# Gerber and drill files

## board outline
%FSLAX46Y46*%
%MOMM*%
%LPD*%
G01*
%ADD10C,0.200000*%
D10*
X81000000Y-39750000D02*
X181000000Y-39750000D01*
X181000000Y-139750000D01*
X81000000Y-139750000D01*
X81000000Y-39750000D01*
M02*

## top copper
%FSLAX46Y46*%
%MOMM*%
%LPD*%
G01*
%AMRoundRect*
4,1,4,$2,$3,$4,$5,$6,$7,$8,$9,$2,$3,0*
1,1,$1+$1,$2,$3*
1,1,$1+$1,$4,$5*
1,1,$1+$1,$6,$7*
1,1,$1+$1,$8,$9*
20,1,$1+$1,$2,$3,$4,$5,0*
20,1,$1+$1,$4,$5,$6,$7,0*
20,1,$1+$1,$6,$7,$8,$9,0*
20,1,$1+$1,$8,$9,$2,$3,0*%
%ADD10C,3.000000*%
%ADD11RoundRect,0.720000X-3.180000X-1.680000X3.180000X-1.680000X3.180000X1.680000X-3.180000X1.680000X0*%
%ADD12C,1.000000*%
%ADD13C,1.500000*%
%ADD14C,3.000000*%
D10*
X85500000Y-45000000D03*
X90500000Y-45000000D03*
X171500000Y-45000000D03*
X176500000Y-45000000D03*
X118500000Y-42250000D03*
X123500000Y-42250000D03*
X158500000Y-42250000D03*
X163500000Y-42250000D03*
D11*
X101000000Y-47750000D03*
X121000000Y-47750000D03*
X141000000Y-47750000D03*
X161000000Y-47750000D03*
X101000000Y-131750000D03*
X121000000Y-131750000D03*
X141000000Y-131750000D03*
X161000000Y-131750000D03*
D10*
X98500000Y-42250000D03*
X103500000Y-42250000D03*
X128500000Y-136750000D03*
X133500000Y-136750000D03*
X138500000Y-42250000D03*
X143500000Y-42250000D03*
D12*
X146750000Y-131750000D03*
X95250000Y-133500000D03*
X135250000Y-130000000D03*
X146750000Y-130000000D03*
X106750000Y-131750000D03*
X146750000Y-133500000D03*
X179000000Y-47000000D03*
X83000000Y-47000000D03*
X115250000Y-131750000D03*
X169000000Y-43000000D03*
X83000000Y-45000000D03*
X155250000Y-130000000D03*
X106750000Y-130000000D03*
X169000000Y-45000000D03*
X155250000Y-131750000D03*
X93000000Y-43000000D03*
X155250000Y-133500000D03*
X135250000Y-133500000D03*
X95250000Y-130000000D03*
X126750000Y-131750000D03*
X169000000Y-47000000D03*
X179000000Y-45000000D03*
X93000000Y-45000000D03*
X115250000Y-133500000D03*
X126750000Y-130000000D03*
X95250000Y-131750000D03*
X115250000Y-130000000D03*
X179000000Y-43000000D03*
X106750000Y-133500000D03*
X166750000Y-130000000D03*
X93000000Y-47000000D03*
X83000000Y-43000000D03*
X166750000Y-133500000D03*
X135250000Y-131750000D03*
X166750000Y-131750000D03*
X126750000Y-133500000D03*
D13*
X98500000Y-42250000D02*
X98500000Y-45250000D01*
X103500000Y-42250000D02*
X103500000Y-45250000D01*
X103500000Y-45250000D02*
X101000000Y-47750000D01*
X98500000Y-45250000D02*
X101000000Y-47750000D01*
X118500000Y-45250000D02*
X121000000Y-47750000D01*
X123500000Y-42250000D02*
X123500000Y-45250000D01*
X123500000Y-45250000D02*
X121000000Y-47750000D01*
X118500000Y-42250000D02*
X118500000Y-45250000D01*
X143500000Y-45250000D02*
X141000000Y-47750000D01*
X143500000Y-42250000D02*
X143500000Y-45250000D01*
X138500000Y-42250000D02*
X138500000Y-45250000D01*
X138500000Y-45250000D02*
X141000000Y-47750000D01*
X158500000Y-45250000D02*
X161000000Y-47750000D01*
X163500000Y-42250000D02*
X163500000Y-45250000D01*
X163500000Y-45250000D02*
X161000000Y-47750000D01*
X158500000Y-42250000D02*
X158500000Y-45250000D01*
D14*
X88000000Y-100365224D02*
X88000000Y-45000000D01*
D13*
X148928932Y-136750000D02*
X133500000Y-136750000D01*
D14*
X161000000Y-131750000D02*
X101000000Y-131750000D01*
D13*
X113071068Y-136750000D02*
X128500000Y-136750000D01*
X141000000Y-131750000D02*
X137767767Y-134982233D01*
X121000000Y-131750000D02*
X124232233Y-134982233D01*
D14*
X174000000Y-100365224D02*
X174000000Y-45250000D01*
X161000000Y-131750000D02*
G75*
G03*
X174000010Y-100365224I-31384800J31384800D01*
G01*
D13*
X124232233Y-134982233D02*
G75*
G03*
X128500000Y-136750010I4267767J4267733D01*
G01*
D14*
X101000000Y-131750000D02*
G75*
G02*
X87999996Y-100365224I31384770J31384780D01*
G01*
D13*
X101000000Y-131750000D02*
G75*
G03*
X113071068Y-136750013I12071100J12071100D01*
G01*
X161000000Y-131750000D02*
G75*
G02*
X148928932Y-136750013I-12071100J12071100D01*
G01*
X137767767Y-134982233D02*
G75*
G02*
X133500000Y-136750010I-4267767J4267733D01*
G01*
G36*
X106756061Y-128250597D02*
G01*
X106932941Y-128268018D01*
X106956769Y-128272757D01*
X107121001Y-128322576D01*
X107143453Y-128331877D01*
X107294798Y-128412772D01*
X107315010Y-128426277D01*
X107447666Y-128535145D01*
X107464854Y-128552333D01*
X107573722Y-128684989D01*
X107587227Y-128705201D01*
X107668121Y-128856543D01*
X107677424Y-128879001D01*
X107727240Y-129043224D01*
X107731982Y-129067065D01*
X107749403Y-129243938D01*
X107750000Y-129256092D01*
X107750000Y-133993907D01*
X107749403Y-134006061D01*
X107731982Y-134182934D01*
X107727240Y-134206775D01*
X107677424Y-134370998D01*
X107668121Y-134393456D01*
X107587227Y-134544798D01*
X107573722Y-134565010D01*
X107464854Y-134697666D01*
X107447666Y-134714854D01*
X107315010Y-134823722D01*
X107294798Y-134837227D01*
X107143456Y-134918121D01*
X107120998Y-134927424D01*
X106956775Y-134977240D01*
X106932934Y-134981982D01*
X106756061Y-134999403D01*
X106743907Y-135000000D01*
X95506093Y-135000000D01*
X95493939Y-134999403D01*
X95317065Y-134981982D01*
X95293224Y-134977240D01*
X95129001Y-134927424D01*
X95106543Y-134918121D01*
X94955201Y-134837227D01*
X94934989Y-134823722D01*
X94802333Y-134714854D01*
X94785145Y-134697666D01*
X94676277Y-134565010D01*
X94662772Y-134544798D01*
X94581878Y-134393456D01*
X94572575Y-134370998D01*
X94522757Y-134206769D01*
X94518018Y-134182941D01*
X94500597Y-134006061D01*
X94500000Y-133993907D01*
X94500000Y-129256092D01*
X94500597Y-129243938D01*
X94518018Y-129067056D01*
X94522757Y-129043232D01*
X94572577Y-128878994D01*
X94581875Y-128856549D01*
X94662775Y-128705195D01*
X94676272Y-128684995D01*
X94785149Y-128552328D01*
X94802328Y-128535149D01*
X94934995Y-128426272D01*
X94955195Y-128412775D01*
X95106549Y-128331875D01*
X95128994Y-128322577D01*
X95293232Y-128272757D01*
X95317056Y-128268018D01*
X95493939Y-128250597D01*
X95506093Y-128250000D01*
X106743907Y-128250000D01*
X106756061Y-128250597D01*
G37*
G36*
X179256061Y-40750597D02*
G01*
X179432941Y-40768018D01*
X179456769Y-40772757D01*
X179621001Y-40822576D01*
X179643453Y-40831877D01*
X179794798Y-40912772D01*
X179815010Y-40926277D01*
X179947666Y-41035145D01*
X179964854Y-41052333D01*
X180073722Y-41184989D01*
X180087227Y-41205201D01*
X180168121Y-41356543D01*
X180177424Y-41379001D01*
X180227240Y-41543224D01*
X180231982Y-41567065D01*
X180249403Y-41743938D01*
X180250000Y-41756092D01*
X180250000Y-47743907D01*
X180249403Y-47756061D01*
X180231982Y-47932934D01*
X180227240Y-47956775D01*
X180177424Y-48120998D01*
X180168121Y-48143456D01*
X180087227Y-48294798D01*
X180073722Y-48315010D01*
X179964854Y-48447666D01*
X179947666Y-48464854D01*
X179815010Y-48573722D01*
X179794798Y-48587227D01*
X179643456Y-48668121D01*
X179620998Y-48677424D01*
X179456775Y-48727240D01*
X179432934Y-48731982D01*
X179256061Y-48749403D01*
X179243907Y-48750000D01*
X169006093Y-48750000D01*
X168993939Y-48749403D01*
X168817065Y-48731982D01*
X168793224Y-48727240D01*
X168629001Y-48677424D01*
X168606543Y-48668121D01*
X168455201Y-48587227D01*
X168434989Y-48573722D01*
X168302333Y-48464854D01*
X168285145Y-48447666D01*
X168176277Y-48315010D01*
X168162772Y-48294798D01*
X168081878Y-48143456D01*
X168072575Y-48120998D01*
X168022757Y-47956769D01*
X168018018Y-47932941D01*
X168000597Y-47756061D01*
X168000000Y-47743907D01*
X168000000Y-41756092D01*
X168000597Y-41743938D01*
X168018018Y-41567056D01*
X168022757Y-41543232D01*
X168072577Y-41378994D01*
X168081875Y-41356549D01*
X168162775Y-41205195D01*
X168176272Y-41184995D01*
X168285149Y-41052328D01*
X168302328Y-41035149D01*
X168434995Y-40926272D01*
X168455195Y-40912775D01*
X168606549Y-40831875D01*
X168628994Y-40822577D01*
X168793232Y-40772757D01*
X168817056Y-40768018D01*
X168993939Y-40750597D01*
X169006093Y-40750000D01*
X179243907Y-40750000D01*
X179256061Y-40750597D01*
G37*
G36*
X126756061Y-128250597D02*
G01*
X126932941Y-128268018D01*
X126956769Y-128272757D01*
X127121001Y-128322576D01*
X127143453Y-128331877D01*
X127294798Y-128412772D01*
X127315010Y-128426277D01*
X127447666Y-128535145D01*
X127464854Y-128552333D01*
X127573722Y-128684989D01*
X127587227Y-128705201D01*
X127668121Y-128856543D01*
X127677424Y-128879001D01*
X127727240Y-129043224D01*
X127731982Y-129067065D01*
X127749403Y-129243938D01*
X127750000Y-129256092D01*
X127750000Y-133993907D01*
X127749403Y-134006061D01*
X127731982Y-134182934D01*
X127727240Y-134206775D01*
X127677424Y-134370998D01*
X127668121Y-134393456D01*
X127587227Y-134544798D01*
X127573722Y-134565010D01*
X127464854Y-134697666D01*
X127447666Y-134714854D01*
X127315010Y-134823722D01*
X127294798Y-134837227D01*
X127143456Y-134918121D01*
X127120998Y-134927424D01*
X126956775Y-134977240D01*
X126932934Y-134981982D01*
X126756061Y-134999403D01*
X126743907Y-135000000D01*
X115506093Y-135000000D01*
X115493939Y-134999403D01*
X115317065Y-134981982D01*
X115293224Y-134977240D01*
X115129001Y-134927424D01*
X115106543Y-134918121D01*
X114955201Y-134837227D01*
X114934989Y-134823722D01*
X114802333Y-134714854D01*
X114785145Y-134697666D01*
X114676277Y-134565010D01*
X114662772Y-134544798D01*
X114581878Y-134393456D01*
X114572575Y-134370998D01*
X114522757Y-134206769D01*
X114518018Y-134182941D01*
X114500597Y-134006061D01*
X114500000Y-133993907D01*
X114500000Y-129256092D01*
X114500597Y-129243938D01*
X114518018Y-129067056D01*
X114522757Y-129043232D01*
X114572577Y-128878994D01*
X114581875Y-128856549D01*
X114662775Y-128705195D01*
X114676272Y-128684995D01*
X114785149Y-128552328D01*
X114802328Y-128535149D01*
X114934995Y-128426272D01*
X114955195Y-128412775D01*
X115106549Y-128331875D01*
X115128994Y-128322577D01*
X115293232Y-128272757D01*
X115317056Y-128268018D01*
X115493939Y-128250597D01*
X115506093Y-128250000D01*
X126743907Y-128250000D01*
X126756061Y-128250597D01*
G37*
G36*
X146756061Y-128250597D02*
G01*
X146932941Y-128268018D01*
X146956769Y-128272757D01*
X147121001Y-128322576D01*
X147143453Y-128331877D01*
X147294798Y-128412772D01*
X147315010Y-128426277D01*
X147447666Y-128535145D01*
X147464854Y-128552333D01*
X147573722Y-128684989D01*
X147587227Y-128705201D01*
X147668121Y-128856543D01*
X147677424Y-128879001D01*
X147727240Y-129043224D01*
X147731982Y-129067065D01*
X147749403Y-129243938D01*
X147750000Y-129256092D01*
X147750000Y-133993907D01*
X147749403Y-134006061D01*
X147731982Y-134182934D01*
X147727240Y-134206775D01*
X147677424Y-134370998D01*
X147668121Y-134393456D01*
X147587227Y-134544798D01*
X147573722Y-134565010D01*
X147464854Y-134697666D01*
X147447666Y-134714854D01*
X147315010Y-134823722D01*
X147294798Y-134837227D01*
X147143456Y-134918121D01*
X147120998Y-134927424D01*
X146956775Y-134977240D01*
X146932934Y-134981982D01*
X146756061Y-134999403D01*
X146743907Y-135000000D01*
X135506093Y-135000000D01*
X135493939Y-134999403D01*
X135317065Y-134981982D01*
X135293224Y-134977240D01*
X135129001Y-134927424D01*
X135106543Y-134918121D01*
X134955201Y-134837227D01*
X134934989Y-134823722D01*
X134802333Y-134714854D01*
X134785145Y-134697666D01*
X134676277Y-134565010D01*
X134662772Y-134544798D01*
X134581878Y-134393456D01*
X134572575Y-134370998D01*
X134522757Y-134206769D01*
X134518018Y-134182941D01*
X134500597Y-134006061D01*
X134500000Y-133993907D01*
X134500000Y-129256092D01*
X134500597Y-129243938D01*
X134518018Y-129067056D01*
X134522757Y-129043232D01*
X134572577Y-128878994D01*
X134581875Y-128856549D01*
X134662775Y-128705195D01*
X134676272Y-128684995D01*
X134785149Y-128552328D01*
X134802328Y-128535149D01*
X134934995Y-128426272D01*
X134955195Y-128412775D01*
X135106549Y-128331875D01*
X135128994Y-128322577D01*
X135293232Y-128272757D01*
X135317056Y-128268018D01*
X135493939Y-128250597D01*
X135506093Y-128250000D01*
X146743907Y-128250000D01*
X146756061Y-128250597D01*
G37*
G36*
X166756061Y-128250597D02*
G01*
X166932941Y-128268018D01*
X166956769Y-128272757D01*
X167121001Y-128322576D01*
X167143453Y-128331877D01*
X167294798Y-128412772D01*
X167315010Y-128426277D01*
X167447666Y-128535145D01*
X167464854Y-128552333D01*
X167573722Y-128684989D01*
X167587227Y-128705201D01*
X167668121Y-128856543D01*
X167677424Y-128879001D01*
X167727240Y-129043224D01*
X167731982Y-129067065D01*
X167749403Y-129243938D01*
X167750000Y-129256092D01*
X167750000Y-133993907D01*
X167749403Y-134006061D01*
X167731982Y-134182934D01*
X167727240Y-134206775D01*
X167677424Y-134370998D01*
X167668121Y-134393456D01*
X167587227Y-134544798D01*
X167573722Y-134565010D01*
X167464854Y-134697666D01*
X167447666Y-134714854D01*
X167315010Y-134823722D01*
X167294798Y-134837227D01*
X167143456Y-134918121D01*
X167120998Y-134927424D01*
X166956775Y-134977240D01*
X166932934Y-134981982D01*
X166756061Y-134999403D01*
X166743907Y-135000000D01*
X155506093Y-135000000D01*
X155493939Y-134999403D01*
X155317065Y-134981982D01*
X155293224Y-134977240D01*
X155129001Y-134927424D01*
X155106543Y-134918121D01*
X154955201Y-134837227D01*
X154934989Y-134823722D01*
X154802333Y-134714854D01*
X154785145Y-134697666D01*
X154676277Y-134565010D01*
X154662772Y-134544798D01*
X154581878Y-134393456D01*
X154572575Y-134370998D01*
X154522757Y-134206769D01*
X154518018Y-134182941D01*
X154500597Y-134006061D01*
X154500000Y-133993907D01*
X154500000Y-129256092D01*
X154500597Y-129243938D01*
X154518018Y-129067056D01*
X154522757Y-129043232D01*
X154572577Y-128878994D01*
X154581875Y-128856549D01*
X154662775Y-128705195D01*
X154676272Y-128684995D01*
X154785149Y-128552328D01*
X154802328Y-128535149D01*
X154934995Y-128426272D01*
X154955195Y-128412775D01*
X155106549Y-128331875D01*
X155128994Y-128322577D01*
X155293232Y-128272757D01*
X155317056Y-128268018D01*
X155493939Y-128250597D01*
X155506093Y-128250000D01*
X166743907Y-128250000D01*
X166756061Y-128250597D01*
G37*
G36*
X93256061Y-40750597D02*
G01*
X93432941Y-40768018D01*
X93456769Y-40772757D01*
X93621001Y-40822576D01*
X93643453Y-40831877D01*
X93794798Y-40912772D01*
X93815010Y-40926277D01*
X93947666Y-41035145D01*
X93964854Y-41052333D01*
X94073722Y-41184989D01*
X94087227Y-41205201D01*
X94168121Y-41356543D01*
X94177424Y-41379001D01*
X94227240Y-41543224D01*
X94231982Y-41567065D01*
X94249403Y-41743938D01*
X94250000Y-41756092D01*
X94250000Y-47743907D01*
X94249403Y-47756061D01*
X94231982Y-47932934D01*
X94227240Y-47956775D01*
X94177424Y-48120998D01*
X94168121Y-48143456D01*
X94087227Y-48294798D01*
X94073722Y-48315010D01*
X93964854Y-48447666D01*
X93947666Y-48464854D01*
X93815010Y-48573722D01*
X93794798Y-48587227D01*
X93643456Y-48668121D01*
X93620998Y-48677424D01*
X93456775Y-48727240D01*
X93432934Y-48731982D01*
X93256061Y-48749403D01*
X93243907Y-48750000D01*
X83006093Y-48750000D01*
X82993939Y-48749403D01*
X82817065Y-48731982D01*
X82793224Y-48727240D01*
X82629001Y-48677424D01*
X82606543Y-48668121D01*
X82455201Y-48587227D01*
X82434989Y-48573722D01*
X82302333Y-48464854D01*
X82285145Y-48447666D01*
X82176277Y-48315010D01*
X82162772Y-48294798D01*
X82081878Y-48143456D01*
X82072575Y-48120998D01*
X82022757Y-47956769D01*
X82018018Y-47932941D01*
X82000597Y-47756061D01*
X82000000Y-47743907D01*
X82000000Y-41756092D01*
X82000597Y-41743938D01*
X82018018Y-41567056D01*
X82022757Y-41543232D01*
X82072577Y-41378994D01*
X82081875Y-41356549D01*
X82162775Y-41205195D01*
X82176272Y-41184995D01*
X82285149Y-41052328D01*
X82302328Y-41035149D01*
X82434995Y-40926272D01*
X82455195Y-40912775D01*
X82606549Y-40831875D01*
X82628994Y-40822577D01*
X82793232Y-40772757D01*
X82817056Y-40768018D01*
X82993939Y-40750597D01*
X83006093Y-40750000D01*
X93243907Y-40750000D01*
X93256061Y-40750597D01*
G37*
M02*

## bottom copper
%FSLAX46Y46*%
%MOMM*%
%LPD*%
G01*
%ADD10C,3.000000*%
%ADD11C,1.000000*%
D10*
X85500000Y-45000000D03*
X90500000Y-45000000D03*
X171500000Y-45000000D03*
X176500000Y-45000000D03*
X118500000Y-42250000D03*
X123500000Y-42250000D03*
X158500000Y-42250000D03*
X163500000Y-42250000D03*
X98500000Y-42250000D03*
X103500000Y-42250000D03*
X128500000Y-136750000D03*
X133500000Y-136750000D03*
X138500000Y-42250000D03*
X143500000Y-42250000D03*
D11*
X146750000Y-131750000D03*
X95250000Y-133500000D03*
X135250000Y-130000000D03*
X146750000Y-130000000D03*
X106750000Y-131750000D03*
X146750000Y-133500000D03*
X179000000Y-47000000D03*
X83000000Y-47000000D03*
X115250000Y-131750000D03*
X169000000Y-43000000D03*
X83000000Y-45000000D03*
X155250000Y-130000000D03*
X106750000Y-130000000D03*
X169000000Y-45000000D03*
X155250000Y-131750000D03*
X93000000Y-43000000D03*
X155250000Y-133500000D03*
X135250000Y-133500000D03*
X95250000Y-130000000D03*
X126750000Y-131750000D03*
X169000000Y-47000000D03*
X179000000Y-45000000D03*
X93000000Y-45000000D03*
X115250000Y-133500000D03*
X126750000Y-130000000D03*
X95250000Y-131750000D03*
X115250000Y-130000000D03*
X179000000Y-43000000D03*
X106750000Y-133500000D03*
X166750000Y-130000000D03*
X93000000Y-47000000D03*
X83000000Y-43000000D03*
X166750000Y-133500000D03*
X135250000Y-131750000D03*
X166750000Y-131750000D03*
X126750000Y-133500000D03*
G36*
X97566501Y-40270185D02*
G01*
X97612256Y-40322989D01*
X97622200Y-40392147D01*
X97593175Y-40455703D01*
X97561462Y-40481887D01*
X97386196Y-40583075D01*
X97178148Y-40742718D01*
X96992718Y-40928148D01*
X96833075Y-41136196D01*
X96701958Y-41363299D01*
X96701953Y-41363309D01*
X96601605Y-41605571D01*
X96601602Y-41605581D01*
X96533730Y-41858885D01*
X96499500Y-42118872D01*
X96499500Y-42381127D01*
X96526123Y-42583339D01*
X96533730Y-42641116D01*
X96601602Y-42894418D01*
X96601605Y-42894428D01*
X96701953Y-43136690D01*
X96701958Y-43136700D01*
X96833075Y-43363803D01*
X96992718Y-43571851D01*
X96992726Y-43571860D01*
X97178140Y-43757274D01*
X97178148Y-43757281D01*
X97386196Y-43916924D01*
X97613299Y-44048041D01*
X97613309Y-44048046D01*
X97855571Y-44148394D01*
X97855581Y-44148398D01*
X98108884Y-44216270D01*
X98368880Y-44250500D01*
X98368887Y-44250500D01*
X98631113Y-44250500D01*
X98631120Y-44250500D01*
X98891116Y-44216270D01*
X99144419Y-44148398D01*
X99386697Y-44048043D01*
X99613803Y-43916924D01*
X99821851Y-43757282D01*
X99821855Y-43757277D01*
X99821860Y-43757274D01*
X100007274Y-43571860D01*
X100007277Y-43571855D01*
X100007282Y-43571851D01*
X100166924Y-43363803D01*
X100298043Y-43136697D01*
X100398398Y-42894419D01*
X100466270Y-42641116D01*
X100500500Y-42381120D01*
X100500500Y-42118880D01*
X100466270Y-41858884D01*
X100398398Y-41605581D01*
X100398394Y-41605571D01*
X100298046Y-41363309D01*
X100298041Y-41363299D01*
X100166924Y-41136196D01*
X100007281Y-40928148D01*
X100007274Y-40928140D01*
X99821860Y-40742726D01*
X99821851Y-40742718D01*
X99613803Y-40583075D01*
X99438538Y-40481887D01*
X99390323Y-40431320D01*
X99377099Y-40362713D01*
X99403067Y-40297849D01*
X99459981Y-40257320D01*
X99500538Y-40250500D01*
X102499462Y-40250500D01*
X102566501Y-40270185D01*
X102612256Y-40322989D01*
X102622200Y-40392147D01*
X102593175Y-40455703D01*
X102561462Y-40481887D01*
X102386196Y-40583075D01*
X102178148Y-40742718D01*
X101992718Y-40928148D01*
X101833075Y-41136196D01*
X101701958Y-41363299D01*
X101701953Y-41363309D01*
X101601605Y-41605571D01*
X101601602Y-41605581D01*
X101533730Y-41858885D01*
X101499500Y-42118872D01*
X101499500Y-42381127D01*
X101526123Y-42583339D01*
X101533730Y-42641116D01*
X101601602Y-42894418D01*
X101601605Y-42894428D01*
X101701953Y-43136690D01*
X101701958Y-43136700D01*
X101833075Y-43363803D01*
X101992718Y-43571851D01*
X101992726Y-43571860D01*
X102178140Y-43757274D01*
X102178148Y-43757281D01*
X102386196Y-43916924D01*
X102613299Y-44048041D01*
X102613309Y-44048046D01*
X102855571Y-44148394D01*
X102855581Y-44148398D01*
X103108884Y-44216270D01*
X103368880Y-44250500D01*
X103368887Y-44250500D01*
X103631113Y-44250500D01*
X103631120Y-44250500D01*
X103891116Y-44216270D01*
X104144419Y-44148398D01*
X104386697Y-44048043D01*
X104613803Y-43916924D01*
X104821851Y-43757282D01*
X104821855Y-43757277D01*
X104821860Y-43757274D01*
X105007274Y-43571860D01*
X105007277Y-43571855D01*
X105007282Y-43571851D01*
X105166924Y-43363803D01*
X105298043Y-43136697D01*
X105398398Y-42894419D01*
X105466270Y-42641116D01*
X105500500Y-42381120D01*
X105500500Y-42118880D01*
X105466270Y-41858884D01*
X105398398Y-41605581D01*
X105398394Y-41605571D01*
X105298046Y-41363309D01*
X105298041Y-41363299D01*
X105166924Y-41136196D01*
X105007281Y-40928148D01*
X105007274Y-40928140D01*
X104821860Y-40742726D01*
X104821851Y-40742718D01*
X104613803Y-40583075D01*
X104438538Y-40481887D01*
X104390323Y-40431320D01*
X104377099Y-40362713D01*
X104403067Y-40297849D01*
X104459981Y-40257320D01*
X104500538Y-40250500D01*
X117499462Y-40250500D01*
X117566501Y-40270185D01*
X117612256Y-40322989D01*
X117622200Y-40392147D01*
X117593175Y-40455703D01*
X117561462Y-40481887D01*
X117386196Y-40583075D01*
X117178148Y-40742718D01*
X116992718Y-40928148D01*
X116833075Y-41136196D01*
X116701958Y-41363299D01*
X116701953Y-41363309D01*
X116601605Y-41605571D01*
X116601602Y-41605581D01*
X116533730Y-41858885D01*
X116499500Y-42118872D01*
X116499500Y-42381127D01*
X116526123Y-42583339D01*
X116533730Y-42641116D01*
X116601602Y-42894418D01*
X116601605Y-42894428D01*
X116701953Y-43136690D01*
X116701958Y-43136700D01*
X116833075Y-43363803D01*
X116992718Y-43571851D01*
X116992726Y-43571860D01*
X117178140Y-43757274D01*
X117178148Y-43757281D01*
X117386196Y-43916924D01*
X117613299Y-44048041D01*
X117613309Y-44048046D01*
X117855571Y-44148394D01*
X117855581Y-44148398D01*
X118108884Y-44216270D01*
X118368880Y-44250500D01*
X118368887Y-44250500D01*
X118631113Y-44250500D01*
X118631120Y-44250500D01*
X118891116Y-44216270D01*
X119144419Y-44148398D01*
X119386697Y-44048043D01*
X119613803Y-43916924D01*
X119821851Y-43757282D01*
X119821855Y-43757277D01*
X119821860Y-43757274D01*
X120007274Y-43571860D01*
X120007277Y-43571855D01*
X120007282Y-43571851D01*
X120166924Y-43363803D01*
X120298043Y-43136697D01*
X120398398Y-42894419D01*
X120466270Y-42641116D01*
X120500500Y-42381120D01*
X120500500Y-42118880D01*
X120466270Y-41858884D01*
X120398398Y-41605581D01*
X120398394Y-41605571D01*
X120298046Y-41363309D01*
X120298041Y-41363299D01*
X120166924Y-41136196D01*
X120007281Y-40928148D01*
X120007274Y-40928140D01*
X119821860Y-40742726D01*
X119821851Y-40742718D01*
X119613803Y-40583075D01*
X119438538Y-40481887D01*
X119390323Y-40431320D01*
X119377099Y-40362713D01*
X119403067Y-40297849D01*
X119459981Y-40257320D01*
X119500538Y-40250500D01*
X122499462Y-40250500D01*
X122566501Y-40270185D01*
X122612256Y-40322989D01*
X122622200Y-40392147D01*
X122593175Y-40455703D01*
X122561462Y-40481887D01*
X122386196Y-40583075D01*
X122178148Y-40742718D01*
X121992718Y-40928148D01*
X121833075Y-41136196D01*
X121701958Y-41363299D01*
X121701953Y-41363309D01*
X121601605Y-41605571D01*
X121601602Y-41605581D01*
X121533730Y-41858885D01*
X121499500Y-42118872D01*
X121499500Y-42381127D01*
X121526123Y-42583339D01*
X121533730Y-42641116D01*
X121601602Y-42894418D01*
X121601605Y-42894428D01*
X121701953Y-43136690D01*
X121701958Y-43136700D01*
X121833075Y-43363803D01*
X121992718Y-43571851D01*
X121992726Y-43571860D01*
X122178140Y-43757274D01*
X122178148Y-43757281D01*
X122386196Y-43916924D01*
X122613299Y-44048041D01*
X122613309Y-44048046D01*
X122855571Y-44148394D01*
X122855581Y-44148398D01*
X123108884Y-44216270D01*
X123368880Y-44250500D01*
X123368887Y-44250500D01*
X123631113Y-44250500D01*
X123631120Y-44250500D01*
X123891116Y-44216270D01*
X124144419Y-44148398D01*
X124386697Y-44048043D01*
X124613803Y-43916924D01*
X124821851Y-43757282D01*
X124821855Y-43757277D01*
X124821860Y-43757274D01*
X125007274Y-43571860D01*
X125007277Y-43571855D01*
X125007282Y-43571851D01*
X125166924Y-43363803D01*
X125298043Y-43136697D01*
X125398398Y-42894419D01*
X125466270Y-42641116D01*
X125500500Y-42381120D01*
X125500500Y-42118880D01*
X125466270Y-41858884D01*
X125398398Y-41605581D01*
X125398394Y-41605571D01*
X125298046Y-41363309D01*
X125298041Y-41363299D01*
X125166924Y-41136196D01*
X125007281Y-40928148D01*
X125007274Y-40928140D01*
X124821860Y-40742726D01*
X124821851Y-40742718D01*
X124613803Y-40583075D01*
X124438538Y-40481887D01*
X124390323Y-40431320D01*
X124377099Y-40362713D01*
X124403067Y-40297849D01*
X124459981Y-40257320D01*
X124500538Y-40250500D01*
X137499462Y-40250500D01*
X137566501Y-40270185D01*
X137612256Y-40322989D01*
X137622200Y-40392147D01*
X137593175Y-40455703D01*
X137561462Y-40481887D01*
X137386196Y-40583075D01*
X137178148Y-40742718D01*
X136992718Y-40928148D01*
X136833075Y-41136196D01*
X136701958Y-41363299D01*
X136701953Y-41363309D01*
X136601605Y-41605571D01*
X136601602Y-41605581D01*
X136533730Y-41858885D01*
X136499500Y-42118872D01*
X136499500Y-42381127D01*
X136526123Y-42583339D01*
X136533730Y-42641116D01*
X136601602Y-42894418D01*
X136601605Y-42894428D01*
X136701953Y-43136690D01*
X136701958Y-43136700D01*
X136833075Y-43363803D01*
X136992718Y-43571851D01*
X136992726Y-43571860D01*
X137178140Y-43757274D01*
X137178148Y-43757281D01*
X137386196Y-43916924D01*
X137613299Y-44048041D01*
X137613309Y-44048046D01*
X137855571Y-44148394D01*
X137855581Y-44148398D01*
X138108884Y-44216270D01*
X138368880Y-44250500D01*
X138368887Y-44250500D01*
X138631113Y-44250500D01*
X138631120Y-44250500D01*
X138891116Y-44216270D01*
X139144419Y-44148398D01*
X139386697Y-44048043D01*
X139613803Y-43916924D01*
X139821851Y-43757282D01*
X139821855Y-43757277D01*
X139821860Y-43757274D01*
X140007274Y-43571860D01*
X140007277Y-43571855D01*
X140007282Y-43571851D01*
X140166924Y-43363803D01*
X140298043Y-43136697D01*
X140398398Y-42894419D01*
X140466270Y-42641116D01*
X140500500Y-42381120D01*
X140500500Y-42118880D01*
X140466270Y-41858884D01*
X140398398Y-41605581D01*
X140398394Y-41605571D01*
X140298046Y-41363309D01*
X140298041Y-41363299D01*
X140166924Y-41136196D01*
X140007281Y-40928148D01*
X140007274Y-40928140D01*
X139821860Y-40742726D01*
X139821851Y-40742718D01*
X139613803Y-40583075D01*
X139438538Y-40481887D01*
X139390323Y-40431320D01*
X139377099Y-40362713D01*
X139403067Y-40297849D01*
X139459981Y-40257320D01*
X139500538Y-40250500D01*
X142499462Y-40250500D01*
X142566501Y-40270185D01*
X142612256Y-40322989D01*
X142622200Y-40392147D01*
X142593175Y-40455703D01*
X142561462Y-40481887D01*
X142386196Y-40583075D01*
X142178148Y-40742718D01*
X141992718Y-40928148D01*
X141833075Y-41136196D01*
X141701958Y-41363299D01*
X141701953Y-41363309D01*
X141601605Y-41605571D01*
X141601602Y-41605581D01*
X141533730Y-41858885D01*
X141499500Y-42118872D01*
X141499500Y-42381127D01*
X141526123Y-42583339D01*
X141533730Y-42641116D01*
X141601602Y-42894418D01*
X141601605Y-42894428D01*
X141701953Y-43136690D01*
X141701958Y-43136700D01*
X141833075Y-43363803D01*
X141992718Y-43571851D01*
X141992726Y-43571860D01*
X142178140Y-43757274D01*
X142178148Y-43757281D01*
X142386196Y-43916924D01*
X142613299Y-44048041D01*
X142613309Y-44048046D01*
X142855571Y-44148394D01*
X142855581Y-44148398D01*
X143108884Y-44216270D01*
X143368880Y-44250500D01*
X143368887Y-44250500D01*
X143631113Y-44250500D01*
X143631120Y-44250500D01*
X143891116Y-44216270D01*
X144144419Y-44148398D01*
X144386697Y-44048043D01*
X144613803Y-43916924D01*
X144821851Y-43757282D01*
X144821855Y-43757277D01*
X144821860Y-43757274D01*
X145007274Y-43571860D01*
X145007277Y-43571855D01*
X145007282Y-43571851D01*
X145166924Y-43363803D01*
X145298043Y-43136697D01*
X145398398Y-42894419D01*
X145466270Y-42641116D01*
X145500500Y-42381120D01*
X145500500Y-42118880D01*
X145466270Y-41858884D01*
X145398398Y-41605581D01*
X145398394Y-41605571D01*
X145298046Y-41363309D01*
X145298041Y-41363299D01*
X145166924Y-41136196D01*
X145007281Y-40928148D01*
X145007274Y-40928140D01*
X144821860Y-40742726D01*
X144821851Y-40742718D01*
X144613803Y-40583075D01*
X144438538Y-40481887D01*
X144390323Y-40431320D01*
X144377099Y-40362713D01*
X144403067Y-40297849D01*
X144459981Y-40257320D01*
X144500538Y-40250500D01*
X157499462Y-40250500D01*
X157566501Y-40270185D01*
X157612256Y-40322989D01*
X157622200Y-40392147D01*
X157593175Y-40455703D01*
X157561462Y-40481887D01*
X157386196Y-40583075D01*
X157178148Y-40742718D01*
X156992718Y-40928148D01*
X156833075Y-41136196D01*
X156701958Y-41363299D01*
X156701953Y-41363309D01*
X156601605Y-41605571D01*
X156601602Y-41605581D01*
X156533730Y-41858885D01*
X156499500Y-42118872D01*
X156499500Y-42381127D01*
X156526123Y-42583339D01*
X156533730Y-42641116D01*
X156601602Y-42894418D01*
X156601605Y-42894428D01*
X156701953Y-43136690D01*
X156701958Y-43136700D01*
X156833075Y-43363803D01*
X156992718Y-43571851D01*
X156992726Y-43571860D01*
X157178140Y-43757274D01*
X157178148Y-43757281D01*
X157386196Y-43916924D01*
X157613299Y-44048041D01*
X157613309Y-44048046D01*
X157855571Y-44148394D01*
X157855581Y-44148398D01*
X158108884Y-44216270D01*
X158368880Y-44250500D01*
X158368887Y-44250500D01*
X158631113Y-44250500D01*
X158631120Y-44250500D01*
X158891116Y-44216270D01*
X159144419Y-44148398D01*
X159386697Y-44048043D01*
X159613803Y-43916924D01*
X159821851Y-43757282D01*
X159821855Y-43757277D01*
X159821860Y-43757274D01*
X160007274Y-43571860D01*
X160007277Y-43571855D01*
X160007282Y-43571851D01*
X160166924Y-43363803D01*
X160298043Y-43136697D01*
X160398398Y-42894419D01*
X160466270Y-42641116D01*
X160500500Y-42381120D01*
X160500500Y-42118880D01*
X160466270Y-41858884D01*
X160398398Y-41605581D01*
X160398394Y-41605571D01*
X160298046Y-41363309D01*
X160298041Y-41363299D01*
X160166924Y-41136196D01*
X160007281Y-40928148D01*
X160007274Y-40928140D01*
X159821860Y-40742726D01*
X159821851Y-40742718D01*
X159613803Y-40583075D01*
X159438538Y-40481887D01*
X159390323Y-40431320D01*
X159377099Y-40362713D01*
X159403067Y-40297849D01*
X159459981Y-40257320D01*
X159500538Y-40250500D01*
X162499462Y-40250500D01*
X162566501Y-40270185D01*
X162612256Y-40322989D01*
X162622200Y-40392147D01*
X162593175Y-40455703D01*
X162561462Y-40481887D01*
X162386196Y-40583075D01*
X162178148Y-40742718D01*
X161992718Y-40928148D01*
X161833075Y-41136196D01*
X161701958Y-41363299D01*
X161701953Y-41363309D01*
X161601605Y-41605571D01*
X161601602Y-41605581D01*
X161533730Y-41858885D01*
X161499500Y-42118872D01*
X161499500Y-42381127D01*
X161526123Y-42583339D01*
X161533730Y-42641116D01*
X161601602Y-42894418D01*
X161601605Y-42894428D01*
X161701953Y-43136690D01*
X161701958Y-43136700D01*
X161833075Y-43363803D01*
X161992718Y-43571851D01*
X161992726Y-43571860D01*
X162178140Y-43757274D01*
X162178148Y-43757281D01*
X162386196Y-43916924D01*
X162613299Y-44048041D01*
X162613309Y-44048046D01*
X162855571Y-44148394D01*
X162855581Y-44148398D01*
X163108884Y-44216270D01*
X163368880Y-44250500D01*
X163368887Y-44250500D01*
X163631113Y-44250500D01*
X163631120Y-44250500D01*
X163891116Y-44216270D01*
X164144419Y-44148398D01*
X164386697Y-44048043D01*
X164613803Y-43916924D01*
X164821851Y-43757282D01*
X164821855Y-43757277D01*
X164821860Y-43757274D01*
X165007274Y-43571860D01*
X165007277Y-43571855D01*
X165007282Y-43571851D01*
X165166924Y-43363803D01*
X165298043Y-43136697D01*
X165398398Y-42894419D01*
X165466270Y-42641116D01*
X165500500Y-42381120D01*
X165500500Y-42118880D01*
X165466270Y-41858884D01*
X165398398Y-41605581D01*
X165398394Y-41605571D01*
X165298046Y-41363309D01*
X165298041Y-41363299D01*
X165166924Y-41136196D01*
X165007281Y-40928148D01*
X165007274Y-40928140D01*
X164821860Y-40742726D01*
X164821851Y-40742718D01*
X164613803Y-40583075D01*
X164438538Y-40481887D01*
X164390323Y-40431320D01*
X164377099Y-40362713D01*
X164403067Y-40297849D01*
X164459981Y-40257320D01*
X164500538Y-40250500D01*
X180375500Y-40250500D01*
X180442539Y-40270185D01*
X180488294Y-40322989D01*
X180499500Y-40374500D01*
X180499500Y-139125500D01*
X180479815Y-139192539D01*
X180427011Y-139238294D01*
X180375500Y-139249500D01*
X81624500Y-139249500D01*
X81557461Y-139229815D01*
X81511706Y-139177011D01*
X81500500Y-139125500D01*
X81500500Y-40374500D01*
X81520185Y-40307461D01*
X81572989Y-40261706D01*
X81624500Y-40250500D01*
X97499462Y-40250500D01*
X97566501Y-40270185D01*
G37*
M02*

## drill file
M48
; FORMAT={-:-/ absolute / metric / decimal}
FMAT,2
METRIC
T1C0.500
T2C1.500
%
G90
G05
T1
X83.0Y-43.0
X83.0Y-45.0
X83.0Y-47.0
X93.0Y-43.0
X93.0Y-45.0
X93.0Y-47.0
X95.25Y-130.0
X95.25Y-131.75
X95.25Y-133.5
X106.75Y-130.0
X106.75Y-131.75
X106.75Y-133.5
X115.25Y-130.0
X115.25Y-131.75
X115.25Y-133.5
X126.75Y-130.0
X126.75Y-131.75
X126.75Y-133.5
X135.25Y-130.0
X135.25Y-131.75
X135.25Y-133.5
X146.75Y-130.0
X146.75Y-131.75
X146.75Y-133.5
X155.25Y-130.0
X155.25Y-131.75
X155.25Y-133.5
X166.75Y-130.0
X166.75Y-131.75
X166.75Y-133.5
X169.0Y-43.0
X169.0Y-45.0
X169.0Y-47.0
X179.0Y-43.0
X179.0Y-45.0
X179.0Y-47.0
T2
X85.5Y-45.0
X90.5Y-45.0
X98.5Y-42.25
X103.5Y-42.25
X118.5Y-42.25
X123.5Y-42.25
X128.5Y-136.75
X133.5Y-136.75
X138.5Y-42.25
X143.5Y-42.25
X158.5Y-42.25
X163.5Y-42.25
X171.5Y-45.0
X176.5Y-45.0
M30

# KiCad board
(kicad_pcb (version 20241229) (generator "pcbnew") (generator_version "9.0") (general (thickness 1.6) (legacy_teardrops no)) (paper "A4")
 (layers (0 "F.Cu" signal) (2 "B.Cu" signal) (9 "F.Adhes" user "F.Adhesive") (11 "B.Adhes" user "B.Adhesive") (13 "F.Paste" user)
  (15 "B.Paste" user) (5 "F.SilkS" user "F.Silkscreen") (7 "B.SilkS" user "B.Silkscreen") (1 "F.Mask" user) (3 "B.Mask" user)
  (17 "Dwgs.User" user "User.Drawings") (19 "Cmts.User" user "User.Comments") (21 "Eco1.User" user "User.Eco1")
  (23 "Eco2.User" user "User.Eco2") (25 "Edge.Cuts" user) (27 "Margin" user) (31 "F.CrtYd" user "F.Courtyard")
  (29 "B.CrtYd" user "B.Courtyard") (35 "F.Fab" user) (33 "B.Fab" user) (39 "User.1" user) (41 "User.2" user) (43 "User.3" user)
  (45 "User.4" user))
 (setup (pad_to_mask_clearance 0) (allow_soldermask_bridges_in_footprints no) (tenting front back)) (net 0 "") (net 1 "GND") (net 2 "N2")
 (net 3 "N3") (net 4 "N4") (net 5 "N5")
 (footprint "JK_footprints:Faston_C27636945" (layer "F.Cu") (at 85.5 45)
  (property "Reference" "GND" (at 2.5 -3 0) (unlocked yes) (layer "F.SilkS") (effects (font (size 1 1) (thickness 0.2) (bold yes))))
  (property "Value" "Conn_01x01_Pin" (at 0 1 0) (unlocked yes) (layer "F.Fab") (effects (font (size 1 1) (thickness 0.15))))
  (pad "1" thru_hole circle (at 0 0) (size 3 3) (drill 1.5) (layers "*.Cu" "*.Mask") (remove_unused_layers no) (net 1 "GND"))
  (pad "1" thru_hole circle (at 5 0) (size 3 3) (drill 1.5) (layers "*.Cu" "*.Mask") (remove_unused_layers no) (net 1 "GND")))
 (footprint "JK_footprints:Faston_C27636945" (layer "F.Cu") (at 171.5 45)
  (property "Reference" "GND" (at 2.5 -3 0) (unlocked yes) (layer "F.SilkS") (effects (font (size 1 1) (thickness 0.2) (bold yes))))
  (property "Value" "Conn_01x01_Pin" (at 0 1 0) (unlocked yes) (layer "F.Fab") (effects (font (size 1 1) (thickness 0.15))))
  (pad "1" thru_hole circle (at 0 0) (size 3 3) (drill 1.5) (layers "*.Cu" "*.Mask") (remove_unused_layers no) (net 1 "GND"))
  (pad "1" thru_hole circle (at 5 0) (size 3 3) (drill 1.5) (layers "*.Cu" "*.Mask") (remove_unused_layers no) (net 1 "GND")))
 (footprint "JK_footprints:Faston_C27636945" (layer "F.Cu") (at 118.5 42.25)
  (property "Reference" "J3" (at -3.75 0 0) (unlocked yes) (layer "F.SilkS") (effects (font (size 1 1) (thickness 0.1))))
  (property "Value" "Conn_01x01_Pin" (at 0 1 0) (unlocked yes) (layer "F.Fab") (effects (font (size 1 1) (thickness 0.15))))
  (pad "1" thru_hole circle (at 0 0) (size 3 3) (drill 1.5) (layers "*.Cu" "*.Mask") (remove_unused_layers no) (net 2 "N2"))
  (pad "1" thru_hole circle (at 5 0) (size 3 3) (drill 1.5) (layers "*.Cu" "*.Mask") (remove_unused_layers no) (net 2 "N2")))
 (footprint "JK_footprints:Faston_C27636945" (layer "F.Cu") (at 158.5 42.25)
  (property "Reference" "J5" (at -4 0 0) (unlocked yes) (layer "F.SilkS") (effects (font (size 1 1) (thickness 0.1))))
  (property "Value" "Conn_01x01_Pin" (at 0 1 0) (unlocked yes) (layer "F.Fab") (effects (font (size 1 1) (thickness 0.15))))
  (pad "1" thru_hole circle (at 0 0) (size 3 3) (drill 1.5) (layers "*.Cu" "*.Mask") (remove_unused_layers no) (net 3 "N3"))
  (pad "1" thru_hole circle (at 5 0) (size 3 3) (drill 1.5) (layers "*.Cu" "*.Mask") (remove_unused_layers no) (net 3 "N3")))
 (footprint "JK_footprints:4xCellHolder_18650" (layer "F.Cu") (at 131 89.75)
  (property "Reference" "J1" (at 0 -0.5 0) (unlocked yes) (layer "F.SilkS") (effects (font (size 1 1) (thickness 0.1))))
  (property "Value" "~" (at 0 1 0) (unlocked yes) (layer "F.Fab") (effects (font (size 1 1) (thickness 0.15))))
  (pad "1" smd roundrect (at -30 -42) (size 7.8 4.8) (layers "F.Cu" "F.Mask") (roundrect_rratio 0.15) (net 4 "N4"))
  (pad "2" smd roundrect (at -10 -42) (size 7.8 4.8) (layers "F.Cu" "F.Mask") (roundrect_rratio 0.15) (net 2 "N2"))
  (pad "3" smd roundrect (at 10 -42) (size 7.8 4.8) (layers "F.Cu" "F.Mask") (roundrect_rratio 0.15) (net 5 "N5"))
  (pad "4" smd roundrect (at 30 -42) (size 7.8 4.8) (layers "F.Cu" "F.Mask") (roundrect_rratio 0.15) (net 3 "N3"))
  (pad "5" smd roundrect (at -30 42) (size 7.8 4.8) (layers "F.Cu" "F.Mask") (roundrect_rratio 0.15) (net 1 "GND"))
  (pad "6" smd roundrect (at -10 42) (size 7.8 4.8) (layers "F.Cu" "F.Mask") (roundrect_rratio 0.15) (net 1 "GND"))
  (pad "7" smd roundrect (at 10 42) (size 7.8 4.8) (layers "F.Cu" "F.Mask") (roundrect_rratio 0.15) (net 1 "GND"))
  (pad "8" smd roundrect (at 30 42) (size 7.8 4.8) (layers "F.Cu" "F.Mask") (roundrect_rratio 0.15) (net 1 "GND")))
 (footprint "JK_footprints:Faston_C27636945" (layer "F.Cu") (at 98.5 42.25)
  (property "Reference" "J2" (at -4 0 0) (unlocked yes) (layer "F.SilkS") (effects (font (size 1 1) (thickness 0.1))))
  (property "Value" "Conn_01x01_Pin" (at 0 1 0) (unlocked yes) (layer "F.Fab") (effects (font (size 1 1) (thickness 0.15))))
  (pad "1" thru_hole circle (at 0 0) (size 3 3) (drill 1.5) (layers "*.Cu" "*.Mask") (remove_unused_layers no) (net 4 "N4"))
  (pad "1" thru_hole circle (at 5 0) (size 3 3) (drill 1.5) (layers "*.Cu" "*.Mask") (remove_unused_layers no) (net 4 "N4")))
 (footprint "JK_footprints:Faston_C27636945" (layer "F.Cu") (at 128.5 136.75)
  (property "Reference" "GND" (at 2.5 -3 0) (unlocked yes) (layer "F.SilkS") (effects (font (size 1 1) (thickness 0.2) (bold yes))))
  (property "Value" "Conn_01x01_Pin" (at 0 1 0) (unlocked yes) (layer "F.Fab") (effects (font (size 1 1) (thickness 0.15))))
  (pad "1" thru_hole circle (at 0 0) (size 3 3) (drill 1.5) (layers "*.Cu" "*.Mask") (remove_unused_layers no) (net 1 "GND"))
  (pad "1" thru_hole circle (at 5 0) (size 3 3) (drill 1.5) (layers "*.Cu" "*.Mask") (remove_unused_layers no) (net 1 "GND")))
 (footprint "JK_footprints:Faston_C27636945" (layer "F.Cu") (at 138.5 42.25)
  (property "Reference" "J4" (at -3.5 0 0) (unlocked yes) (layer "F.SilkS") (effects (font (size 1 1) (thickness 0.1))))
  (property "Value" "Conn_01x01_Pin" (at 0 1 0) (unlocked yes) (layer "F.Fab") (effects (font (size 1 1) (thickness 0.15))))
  (pad "1" thru_hole circle (at 0 0) (size 3 3) (drill 1.5) (layers "*.Cu" "*.Mask") (remove_unused_layers no) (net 5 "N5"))
  (pad "1" thru_hole circle (at 5 0) (size 3 3) (drill 1.5) (layers "*.Cu" "*.Mask") (remove_unused_layers no) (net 5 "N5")))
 (gr_rect (start 81 39.75) (end 181 139.75) (stroke (width 0.2) (type solid)) (fill no) (layer "Edge.Cuts"))
 (segment (start 98.5 42.25) (end 98.5 45.25) (width 1.5) (layer "F.Cu") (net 4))
 (segment (start 103.5 42.25) (end 103.5 45.25) (width 1.5) (layer "F.Cu") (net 4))
 (segment (start 103.5 45.25) (end 101 47.75) (width 1.5) (layer "F.Cu") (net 4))
 (segment (start 98.5 45.25) (end 101 47.75) (width 1.5) (layer "F.Cu") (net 4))
 (segment (start 118.5 45.25) (end 121 47.75) (width 1.5) (layer "F.Cu") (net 2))
 (segment (start 123.5 42.25) (end 123.5 45.25) (width 1.5) (layer "F.Cu") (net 2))
 (segment (start 123.5 45.25) (end 121 47.75) (width 1.5) (layer "F.Cu") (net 2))
 (segment (start 118.5 42.25) (end 118.5 45.25) (width 1.5) (layer "F.Cu") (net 2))
 (segment (start 143.5 45.25) (end 141 47.75) (width 1.5) (layer "F.Cu") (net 5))
 (segment (start 143.5 42.25) (end 143.5 45.25) (width 1.5) (layer "F.Cu") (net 5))
 (segment (start 138.5 42.25) (end 138.5 45.25) (width 1.5) (layer "F.Cu") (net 5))
 (segment (start 138.5 45.25) (end 141 47.75) (width 1.5) (layer "F.Cu") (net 5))
 (segment (start 158.5 45.25) (end 161 47.75) (width 1.5) (layer "F.Cu") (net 3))
 (segment (start 163.5 42.25) (end 163.5 45.25) (width 1.5) (layer "F.Cu") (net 3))
 (segment (start 163.5 45.25) (end 161 47.75) (width 1.5) (layer "F.Cu") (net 3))
 (segment (start 158.5 42.25) (end 158.5 45.25) (width 1.5) (layer "F.Cu") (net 3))
 (segment (start 88 100.365224) (end 88 45) (width 3) (layer "F.Cu") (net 1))
 (segment (start 148.928932 136.75) (end 133.5 136.75) (width 1.5) (layer "F.Cu") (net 1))
 (segment (start 161 131.75) (end 101 131.75) (width 3) (layer "F.Cu") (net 1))
 (segment (start 113.071068 136.75) (end 128.5 136.75) (width 1.5) (layer "F.Cu") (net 1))
 (segment (start 141 131.75) (end 137.767767 134.982233) (width 1.5) (layer "F.Cu") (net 1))
 (segment (start 121 131.75) (end 124.232233 134.982233) (width 1.5) (layer "F.Cu") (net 1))
 (segment (start 174 100.365224) (end 174 45.25) (width 3) (layer "F.Cu") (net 1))
 (via (at 146.75 131.75) (size 1) (drill 0.5) (layers "F.Cu" "B.Cu") (free yes) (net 1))
 (via (at 95.25 133.5) (size 1) (drill 0.5) (layers "F.Cu" "B.Cu") (free yes) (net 1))
 (via (at 135.25 130) (size 1) (drill 0.5) (layers "F.Cu" "B.Cu") (free yes) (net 1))
 (via (at 146.75 130) (size 1) (drill 0.5) (layers "F.Cu" "B.Cu") (free yes) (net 1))
 (via (at 106.75 131.75) (size 1) (drill 0.5) (layers "F.Cu" "B.Cu") (free yes) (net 1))
 (via (at 146.75 133.5) (size 1) (drill 0.5) (layers "F.Cu" "B.Cu") (free yes) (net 1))
 (via (at 179 47) (size 1) (drill 0.5) (layers "F.Cu" "B.Cu") (free yes) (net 1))
 (via (at 83 47) (size 1) (drill 0.5) (layers "F.Cu" "B.Cu") (free yes) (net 1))
 (via (at 115.25 131.75) (size 1) (drill 0.5) (layers "F.Cu" "B.Cu") (free yes) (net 1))
 (via (at 169 43) (size 1) (drill 0.5) (layers "F.Cu" "B.Cu") (free yes) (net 1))
 (via (at 83 45) (size 1) (drill 0.5) (layers "F.Cu" "B.Cu") (free yes) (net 1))
 (via (at 155.25 130) (size 1) (drill 0.5) (layers "F.Cu" "B.Cu") (free yes) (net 1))
 (via (at 106.75 130) (size 1) (drill 0.5) (layers "F.Cu" "B.Cu") (free yes) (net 1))
 (via (at 169 45) (size 1) (drill 0.5) (layers "F.Cu" "B.Cu") (free yes) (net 1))
 (via (at 155.25 131.75) (size 1) (drill 0.5) (layers "F.Cu" "B.Cu") (free yes) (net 1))
 (via (at 93 43) (size 1) (drill 0.5) (layers "F.Cu" "B.Cu") (free yes) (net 1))
 (via (at 155.25 133.5) (size 1) (drill 0.5) (layers "F.Cu" "B.Cu") (free yes) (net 1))
 (via (at 135.25 133.5) (size 1) (drill 0.5) (layers "F.Cu" "B.Cu") (free yes) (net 1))
 (via (at 95.25 130) (size 1) (drill 0.5) (layers "F.Cu" "B.Cu") (free yes) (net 1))
 (via (at 126.75 131.75) (size 1) (drill 0.5) (layers "F.Cu" "B.Cu") (free yes) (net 1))
 (via (at 169 47) (size 1) (drill 0.5) (layers "F.Cu" "B.Cu") (free yes) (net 1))
 (via (at 179 45) (size 1) (drill 0.5) (layers "F.Cu" "B.Cu") (free yes) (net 1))
 (via (at 93 45) (size 1) (drill 0.5) (layers "F.Cu" "B.Cu") (free yes) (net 1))
 (via (at 115.25 133.5) (size 1) (drill 0.5) (layers "F.Cu" "B.Cu") (free yes) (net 1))
 (via (at 126.75 130) (size 1) (drill 0.5) (layers "F.Cu" "B.Cu") (free yes) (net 1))
 (via (at 95.25 131.75) (size 1) (drill 0.5) (layers "F.Cu" "B.Cu") (free yes) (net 1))
 (via (at 115.25 130) (size 1) (drill 0.5) (layers "F.Cu" "B.Cu") (free yes) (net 1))
 (via (at 179 43) (size 1) (drill 0.5) (layers "F.Cu" "B.Cu") (free yes) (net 1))
 (via (at 106.75 133.5) (size 1) (drill 0.5) (layers "F.Cu" "B.Cu") (free yes) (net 1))
 (via (at 166.75 130) (size 1) (drill 0.5) (layers "F.Cu" "B.Cu") (free yes) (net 1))
 (via (at 93 47) (size 1) (drill 0.5) (layers "F.Cu" "B.Cu") (free yes) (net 1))
 (via (at 83 43) (size 1) (drill 0.5) (layers "F.Cu" "B.Cu") (free yes) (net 1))
 (via (at 166.75 133.5) (size 1) (drill 0.5) (layers "F.Cu" "B.Cu") (free yes) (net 1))
 (via (at 135.25 131.75) (size 1) (drill 0.5) (layers "F.Cu" "B.Cu") (free yes) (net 1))
 (via (at 166.75 131.75) (size 1) (drill 0.5) (layers "F.Cu" "B.Cu") (free yes) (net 1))
 (via (at 126.75 133.5) (size 1) (drill 0.5) (layers "F.Cu" "B.Cu") (free yes) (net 1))
 (arc (start 161 131.75) (mid 170.62141 117.350542) (end 174 100.365224) (width 3) (layer "F.Cu") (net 1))
 (arc (start 124.232233 134.982233) (mid 126.190301 136.290572) (end 128.5 136.75) (width 1.5) (layer "F.Cu") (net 1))
 (arc (start 101 131.75) (mid 91.37859 117.350543) (end 88 100.365224) (width 3) (layer "F.Cu") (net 1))
 (arc (start 101 131.75) (mid 106.538253 135.450542) (end 113.071068 136.75) (width 1.5) (layer "F.Cu") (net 1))
 (arc (start 161 131.75) (mid 155.461747 135.450542) (end 148.928932 136.75) (width 1.5) (layer "F.Cu") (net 1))
 (arc (start 137.767767 134.982233) (mid 135.809699 136.290573) (end 133.5 136.75) (width 1.5) (layer "F.Cu") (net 1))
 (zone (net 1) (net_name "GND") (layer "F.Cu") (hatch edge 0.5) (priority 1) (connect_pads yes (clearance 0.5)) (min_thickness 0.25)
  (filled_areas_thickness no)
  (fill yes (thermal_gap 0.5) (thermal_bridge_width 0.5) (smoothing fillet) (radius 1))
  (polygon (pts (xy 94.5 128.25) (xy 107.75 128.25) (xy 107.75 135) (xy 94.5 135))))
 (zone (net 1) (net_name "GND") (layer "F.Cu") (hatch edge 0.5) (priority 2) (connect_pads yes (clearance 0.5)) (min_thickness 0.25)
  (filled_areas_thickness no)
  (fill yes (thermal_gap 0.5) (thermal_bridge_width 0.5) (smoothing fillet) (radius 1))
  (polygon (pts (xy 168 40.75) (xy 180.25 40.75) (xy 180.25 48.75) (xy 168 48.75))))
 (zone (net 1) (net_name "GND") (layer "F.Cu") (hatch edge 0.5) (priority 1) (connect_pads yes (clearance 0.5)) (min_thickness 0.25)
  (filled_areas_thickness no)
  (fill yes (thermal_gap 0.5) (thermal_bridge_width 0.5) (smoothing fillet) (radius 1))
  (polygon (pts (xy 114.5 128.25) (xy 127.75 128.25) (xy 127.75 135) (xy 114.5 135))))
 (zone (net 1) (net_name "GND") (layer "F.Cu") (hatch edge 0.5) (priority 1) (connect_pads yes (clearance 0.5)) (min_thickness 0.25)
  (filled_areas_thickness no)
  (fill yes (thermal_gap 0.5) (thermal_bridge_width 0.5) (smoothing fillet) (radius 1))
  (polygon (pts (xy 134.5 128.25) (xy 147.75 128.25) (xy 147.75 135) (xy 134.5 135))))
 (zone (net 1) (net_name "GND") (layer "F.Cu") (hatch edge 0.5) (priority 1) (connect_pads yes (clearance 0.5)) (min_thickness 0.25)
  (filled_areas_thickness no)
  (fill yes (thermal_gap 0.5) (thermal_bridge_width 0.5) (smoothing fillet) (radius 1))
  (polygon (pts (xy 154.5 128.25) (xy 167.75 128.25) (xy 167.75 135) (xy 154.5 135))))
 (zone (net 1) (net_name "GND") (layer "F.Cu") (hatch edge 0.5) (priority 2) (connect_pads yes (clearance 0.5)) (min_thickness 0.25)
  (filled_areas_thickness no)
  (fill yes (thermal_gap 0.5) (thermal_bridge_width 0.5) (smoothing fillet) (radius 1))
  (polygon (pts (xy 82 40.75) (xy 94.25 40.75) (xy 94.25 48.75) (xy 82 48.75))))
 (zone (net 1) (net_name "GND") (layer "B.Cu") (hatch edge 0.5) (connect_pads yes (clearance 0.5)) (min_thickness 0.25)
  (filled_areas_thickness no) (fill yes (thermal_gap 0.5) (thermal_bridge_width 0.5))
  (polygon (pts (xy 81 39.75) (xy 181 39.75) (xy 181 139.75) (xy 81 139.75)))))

